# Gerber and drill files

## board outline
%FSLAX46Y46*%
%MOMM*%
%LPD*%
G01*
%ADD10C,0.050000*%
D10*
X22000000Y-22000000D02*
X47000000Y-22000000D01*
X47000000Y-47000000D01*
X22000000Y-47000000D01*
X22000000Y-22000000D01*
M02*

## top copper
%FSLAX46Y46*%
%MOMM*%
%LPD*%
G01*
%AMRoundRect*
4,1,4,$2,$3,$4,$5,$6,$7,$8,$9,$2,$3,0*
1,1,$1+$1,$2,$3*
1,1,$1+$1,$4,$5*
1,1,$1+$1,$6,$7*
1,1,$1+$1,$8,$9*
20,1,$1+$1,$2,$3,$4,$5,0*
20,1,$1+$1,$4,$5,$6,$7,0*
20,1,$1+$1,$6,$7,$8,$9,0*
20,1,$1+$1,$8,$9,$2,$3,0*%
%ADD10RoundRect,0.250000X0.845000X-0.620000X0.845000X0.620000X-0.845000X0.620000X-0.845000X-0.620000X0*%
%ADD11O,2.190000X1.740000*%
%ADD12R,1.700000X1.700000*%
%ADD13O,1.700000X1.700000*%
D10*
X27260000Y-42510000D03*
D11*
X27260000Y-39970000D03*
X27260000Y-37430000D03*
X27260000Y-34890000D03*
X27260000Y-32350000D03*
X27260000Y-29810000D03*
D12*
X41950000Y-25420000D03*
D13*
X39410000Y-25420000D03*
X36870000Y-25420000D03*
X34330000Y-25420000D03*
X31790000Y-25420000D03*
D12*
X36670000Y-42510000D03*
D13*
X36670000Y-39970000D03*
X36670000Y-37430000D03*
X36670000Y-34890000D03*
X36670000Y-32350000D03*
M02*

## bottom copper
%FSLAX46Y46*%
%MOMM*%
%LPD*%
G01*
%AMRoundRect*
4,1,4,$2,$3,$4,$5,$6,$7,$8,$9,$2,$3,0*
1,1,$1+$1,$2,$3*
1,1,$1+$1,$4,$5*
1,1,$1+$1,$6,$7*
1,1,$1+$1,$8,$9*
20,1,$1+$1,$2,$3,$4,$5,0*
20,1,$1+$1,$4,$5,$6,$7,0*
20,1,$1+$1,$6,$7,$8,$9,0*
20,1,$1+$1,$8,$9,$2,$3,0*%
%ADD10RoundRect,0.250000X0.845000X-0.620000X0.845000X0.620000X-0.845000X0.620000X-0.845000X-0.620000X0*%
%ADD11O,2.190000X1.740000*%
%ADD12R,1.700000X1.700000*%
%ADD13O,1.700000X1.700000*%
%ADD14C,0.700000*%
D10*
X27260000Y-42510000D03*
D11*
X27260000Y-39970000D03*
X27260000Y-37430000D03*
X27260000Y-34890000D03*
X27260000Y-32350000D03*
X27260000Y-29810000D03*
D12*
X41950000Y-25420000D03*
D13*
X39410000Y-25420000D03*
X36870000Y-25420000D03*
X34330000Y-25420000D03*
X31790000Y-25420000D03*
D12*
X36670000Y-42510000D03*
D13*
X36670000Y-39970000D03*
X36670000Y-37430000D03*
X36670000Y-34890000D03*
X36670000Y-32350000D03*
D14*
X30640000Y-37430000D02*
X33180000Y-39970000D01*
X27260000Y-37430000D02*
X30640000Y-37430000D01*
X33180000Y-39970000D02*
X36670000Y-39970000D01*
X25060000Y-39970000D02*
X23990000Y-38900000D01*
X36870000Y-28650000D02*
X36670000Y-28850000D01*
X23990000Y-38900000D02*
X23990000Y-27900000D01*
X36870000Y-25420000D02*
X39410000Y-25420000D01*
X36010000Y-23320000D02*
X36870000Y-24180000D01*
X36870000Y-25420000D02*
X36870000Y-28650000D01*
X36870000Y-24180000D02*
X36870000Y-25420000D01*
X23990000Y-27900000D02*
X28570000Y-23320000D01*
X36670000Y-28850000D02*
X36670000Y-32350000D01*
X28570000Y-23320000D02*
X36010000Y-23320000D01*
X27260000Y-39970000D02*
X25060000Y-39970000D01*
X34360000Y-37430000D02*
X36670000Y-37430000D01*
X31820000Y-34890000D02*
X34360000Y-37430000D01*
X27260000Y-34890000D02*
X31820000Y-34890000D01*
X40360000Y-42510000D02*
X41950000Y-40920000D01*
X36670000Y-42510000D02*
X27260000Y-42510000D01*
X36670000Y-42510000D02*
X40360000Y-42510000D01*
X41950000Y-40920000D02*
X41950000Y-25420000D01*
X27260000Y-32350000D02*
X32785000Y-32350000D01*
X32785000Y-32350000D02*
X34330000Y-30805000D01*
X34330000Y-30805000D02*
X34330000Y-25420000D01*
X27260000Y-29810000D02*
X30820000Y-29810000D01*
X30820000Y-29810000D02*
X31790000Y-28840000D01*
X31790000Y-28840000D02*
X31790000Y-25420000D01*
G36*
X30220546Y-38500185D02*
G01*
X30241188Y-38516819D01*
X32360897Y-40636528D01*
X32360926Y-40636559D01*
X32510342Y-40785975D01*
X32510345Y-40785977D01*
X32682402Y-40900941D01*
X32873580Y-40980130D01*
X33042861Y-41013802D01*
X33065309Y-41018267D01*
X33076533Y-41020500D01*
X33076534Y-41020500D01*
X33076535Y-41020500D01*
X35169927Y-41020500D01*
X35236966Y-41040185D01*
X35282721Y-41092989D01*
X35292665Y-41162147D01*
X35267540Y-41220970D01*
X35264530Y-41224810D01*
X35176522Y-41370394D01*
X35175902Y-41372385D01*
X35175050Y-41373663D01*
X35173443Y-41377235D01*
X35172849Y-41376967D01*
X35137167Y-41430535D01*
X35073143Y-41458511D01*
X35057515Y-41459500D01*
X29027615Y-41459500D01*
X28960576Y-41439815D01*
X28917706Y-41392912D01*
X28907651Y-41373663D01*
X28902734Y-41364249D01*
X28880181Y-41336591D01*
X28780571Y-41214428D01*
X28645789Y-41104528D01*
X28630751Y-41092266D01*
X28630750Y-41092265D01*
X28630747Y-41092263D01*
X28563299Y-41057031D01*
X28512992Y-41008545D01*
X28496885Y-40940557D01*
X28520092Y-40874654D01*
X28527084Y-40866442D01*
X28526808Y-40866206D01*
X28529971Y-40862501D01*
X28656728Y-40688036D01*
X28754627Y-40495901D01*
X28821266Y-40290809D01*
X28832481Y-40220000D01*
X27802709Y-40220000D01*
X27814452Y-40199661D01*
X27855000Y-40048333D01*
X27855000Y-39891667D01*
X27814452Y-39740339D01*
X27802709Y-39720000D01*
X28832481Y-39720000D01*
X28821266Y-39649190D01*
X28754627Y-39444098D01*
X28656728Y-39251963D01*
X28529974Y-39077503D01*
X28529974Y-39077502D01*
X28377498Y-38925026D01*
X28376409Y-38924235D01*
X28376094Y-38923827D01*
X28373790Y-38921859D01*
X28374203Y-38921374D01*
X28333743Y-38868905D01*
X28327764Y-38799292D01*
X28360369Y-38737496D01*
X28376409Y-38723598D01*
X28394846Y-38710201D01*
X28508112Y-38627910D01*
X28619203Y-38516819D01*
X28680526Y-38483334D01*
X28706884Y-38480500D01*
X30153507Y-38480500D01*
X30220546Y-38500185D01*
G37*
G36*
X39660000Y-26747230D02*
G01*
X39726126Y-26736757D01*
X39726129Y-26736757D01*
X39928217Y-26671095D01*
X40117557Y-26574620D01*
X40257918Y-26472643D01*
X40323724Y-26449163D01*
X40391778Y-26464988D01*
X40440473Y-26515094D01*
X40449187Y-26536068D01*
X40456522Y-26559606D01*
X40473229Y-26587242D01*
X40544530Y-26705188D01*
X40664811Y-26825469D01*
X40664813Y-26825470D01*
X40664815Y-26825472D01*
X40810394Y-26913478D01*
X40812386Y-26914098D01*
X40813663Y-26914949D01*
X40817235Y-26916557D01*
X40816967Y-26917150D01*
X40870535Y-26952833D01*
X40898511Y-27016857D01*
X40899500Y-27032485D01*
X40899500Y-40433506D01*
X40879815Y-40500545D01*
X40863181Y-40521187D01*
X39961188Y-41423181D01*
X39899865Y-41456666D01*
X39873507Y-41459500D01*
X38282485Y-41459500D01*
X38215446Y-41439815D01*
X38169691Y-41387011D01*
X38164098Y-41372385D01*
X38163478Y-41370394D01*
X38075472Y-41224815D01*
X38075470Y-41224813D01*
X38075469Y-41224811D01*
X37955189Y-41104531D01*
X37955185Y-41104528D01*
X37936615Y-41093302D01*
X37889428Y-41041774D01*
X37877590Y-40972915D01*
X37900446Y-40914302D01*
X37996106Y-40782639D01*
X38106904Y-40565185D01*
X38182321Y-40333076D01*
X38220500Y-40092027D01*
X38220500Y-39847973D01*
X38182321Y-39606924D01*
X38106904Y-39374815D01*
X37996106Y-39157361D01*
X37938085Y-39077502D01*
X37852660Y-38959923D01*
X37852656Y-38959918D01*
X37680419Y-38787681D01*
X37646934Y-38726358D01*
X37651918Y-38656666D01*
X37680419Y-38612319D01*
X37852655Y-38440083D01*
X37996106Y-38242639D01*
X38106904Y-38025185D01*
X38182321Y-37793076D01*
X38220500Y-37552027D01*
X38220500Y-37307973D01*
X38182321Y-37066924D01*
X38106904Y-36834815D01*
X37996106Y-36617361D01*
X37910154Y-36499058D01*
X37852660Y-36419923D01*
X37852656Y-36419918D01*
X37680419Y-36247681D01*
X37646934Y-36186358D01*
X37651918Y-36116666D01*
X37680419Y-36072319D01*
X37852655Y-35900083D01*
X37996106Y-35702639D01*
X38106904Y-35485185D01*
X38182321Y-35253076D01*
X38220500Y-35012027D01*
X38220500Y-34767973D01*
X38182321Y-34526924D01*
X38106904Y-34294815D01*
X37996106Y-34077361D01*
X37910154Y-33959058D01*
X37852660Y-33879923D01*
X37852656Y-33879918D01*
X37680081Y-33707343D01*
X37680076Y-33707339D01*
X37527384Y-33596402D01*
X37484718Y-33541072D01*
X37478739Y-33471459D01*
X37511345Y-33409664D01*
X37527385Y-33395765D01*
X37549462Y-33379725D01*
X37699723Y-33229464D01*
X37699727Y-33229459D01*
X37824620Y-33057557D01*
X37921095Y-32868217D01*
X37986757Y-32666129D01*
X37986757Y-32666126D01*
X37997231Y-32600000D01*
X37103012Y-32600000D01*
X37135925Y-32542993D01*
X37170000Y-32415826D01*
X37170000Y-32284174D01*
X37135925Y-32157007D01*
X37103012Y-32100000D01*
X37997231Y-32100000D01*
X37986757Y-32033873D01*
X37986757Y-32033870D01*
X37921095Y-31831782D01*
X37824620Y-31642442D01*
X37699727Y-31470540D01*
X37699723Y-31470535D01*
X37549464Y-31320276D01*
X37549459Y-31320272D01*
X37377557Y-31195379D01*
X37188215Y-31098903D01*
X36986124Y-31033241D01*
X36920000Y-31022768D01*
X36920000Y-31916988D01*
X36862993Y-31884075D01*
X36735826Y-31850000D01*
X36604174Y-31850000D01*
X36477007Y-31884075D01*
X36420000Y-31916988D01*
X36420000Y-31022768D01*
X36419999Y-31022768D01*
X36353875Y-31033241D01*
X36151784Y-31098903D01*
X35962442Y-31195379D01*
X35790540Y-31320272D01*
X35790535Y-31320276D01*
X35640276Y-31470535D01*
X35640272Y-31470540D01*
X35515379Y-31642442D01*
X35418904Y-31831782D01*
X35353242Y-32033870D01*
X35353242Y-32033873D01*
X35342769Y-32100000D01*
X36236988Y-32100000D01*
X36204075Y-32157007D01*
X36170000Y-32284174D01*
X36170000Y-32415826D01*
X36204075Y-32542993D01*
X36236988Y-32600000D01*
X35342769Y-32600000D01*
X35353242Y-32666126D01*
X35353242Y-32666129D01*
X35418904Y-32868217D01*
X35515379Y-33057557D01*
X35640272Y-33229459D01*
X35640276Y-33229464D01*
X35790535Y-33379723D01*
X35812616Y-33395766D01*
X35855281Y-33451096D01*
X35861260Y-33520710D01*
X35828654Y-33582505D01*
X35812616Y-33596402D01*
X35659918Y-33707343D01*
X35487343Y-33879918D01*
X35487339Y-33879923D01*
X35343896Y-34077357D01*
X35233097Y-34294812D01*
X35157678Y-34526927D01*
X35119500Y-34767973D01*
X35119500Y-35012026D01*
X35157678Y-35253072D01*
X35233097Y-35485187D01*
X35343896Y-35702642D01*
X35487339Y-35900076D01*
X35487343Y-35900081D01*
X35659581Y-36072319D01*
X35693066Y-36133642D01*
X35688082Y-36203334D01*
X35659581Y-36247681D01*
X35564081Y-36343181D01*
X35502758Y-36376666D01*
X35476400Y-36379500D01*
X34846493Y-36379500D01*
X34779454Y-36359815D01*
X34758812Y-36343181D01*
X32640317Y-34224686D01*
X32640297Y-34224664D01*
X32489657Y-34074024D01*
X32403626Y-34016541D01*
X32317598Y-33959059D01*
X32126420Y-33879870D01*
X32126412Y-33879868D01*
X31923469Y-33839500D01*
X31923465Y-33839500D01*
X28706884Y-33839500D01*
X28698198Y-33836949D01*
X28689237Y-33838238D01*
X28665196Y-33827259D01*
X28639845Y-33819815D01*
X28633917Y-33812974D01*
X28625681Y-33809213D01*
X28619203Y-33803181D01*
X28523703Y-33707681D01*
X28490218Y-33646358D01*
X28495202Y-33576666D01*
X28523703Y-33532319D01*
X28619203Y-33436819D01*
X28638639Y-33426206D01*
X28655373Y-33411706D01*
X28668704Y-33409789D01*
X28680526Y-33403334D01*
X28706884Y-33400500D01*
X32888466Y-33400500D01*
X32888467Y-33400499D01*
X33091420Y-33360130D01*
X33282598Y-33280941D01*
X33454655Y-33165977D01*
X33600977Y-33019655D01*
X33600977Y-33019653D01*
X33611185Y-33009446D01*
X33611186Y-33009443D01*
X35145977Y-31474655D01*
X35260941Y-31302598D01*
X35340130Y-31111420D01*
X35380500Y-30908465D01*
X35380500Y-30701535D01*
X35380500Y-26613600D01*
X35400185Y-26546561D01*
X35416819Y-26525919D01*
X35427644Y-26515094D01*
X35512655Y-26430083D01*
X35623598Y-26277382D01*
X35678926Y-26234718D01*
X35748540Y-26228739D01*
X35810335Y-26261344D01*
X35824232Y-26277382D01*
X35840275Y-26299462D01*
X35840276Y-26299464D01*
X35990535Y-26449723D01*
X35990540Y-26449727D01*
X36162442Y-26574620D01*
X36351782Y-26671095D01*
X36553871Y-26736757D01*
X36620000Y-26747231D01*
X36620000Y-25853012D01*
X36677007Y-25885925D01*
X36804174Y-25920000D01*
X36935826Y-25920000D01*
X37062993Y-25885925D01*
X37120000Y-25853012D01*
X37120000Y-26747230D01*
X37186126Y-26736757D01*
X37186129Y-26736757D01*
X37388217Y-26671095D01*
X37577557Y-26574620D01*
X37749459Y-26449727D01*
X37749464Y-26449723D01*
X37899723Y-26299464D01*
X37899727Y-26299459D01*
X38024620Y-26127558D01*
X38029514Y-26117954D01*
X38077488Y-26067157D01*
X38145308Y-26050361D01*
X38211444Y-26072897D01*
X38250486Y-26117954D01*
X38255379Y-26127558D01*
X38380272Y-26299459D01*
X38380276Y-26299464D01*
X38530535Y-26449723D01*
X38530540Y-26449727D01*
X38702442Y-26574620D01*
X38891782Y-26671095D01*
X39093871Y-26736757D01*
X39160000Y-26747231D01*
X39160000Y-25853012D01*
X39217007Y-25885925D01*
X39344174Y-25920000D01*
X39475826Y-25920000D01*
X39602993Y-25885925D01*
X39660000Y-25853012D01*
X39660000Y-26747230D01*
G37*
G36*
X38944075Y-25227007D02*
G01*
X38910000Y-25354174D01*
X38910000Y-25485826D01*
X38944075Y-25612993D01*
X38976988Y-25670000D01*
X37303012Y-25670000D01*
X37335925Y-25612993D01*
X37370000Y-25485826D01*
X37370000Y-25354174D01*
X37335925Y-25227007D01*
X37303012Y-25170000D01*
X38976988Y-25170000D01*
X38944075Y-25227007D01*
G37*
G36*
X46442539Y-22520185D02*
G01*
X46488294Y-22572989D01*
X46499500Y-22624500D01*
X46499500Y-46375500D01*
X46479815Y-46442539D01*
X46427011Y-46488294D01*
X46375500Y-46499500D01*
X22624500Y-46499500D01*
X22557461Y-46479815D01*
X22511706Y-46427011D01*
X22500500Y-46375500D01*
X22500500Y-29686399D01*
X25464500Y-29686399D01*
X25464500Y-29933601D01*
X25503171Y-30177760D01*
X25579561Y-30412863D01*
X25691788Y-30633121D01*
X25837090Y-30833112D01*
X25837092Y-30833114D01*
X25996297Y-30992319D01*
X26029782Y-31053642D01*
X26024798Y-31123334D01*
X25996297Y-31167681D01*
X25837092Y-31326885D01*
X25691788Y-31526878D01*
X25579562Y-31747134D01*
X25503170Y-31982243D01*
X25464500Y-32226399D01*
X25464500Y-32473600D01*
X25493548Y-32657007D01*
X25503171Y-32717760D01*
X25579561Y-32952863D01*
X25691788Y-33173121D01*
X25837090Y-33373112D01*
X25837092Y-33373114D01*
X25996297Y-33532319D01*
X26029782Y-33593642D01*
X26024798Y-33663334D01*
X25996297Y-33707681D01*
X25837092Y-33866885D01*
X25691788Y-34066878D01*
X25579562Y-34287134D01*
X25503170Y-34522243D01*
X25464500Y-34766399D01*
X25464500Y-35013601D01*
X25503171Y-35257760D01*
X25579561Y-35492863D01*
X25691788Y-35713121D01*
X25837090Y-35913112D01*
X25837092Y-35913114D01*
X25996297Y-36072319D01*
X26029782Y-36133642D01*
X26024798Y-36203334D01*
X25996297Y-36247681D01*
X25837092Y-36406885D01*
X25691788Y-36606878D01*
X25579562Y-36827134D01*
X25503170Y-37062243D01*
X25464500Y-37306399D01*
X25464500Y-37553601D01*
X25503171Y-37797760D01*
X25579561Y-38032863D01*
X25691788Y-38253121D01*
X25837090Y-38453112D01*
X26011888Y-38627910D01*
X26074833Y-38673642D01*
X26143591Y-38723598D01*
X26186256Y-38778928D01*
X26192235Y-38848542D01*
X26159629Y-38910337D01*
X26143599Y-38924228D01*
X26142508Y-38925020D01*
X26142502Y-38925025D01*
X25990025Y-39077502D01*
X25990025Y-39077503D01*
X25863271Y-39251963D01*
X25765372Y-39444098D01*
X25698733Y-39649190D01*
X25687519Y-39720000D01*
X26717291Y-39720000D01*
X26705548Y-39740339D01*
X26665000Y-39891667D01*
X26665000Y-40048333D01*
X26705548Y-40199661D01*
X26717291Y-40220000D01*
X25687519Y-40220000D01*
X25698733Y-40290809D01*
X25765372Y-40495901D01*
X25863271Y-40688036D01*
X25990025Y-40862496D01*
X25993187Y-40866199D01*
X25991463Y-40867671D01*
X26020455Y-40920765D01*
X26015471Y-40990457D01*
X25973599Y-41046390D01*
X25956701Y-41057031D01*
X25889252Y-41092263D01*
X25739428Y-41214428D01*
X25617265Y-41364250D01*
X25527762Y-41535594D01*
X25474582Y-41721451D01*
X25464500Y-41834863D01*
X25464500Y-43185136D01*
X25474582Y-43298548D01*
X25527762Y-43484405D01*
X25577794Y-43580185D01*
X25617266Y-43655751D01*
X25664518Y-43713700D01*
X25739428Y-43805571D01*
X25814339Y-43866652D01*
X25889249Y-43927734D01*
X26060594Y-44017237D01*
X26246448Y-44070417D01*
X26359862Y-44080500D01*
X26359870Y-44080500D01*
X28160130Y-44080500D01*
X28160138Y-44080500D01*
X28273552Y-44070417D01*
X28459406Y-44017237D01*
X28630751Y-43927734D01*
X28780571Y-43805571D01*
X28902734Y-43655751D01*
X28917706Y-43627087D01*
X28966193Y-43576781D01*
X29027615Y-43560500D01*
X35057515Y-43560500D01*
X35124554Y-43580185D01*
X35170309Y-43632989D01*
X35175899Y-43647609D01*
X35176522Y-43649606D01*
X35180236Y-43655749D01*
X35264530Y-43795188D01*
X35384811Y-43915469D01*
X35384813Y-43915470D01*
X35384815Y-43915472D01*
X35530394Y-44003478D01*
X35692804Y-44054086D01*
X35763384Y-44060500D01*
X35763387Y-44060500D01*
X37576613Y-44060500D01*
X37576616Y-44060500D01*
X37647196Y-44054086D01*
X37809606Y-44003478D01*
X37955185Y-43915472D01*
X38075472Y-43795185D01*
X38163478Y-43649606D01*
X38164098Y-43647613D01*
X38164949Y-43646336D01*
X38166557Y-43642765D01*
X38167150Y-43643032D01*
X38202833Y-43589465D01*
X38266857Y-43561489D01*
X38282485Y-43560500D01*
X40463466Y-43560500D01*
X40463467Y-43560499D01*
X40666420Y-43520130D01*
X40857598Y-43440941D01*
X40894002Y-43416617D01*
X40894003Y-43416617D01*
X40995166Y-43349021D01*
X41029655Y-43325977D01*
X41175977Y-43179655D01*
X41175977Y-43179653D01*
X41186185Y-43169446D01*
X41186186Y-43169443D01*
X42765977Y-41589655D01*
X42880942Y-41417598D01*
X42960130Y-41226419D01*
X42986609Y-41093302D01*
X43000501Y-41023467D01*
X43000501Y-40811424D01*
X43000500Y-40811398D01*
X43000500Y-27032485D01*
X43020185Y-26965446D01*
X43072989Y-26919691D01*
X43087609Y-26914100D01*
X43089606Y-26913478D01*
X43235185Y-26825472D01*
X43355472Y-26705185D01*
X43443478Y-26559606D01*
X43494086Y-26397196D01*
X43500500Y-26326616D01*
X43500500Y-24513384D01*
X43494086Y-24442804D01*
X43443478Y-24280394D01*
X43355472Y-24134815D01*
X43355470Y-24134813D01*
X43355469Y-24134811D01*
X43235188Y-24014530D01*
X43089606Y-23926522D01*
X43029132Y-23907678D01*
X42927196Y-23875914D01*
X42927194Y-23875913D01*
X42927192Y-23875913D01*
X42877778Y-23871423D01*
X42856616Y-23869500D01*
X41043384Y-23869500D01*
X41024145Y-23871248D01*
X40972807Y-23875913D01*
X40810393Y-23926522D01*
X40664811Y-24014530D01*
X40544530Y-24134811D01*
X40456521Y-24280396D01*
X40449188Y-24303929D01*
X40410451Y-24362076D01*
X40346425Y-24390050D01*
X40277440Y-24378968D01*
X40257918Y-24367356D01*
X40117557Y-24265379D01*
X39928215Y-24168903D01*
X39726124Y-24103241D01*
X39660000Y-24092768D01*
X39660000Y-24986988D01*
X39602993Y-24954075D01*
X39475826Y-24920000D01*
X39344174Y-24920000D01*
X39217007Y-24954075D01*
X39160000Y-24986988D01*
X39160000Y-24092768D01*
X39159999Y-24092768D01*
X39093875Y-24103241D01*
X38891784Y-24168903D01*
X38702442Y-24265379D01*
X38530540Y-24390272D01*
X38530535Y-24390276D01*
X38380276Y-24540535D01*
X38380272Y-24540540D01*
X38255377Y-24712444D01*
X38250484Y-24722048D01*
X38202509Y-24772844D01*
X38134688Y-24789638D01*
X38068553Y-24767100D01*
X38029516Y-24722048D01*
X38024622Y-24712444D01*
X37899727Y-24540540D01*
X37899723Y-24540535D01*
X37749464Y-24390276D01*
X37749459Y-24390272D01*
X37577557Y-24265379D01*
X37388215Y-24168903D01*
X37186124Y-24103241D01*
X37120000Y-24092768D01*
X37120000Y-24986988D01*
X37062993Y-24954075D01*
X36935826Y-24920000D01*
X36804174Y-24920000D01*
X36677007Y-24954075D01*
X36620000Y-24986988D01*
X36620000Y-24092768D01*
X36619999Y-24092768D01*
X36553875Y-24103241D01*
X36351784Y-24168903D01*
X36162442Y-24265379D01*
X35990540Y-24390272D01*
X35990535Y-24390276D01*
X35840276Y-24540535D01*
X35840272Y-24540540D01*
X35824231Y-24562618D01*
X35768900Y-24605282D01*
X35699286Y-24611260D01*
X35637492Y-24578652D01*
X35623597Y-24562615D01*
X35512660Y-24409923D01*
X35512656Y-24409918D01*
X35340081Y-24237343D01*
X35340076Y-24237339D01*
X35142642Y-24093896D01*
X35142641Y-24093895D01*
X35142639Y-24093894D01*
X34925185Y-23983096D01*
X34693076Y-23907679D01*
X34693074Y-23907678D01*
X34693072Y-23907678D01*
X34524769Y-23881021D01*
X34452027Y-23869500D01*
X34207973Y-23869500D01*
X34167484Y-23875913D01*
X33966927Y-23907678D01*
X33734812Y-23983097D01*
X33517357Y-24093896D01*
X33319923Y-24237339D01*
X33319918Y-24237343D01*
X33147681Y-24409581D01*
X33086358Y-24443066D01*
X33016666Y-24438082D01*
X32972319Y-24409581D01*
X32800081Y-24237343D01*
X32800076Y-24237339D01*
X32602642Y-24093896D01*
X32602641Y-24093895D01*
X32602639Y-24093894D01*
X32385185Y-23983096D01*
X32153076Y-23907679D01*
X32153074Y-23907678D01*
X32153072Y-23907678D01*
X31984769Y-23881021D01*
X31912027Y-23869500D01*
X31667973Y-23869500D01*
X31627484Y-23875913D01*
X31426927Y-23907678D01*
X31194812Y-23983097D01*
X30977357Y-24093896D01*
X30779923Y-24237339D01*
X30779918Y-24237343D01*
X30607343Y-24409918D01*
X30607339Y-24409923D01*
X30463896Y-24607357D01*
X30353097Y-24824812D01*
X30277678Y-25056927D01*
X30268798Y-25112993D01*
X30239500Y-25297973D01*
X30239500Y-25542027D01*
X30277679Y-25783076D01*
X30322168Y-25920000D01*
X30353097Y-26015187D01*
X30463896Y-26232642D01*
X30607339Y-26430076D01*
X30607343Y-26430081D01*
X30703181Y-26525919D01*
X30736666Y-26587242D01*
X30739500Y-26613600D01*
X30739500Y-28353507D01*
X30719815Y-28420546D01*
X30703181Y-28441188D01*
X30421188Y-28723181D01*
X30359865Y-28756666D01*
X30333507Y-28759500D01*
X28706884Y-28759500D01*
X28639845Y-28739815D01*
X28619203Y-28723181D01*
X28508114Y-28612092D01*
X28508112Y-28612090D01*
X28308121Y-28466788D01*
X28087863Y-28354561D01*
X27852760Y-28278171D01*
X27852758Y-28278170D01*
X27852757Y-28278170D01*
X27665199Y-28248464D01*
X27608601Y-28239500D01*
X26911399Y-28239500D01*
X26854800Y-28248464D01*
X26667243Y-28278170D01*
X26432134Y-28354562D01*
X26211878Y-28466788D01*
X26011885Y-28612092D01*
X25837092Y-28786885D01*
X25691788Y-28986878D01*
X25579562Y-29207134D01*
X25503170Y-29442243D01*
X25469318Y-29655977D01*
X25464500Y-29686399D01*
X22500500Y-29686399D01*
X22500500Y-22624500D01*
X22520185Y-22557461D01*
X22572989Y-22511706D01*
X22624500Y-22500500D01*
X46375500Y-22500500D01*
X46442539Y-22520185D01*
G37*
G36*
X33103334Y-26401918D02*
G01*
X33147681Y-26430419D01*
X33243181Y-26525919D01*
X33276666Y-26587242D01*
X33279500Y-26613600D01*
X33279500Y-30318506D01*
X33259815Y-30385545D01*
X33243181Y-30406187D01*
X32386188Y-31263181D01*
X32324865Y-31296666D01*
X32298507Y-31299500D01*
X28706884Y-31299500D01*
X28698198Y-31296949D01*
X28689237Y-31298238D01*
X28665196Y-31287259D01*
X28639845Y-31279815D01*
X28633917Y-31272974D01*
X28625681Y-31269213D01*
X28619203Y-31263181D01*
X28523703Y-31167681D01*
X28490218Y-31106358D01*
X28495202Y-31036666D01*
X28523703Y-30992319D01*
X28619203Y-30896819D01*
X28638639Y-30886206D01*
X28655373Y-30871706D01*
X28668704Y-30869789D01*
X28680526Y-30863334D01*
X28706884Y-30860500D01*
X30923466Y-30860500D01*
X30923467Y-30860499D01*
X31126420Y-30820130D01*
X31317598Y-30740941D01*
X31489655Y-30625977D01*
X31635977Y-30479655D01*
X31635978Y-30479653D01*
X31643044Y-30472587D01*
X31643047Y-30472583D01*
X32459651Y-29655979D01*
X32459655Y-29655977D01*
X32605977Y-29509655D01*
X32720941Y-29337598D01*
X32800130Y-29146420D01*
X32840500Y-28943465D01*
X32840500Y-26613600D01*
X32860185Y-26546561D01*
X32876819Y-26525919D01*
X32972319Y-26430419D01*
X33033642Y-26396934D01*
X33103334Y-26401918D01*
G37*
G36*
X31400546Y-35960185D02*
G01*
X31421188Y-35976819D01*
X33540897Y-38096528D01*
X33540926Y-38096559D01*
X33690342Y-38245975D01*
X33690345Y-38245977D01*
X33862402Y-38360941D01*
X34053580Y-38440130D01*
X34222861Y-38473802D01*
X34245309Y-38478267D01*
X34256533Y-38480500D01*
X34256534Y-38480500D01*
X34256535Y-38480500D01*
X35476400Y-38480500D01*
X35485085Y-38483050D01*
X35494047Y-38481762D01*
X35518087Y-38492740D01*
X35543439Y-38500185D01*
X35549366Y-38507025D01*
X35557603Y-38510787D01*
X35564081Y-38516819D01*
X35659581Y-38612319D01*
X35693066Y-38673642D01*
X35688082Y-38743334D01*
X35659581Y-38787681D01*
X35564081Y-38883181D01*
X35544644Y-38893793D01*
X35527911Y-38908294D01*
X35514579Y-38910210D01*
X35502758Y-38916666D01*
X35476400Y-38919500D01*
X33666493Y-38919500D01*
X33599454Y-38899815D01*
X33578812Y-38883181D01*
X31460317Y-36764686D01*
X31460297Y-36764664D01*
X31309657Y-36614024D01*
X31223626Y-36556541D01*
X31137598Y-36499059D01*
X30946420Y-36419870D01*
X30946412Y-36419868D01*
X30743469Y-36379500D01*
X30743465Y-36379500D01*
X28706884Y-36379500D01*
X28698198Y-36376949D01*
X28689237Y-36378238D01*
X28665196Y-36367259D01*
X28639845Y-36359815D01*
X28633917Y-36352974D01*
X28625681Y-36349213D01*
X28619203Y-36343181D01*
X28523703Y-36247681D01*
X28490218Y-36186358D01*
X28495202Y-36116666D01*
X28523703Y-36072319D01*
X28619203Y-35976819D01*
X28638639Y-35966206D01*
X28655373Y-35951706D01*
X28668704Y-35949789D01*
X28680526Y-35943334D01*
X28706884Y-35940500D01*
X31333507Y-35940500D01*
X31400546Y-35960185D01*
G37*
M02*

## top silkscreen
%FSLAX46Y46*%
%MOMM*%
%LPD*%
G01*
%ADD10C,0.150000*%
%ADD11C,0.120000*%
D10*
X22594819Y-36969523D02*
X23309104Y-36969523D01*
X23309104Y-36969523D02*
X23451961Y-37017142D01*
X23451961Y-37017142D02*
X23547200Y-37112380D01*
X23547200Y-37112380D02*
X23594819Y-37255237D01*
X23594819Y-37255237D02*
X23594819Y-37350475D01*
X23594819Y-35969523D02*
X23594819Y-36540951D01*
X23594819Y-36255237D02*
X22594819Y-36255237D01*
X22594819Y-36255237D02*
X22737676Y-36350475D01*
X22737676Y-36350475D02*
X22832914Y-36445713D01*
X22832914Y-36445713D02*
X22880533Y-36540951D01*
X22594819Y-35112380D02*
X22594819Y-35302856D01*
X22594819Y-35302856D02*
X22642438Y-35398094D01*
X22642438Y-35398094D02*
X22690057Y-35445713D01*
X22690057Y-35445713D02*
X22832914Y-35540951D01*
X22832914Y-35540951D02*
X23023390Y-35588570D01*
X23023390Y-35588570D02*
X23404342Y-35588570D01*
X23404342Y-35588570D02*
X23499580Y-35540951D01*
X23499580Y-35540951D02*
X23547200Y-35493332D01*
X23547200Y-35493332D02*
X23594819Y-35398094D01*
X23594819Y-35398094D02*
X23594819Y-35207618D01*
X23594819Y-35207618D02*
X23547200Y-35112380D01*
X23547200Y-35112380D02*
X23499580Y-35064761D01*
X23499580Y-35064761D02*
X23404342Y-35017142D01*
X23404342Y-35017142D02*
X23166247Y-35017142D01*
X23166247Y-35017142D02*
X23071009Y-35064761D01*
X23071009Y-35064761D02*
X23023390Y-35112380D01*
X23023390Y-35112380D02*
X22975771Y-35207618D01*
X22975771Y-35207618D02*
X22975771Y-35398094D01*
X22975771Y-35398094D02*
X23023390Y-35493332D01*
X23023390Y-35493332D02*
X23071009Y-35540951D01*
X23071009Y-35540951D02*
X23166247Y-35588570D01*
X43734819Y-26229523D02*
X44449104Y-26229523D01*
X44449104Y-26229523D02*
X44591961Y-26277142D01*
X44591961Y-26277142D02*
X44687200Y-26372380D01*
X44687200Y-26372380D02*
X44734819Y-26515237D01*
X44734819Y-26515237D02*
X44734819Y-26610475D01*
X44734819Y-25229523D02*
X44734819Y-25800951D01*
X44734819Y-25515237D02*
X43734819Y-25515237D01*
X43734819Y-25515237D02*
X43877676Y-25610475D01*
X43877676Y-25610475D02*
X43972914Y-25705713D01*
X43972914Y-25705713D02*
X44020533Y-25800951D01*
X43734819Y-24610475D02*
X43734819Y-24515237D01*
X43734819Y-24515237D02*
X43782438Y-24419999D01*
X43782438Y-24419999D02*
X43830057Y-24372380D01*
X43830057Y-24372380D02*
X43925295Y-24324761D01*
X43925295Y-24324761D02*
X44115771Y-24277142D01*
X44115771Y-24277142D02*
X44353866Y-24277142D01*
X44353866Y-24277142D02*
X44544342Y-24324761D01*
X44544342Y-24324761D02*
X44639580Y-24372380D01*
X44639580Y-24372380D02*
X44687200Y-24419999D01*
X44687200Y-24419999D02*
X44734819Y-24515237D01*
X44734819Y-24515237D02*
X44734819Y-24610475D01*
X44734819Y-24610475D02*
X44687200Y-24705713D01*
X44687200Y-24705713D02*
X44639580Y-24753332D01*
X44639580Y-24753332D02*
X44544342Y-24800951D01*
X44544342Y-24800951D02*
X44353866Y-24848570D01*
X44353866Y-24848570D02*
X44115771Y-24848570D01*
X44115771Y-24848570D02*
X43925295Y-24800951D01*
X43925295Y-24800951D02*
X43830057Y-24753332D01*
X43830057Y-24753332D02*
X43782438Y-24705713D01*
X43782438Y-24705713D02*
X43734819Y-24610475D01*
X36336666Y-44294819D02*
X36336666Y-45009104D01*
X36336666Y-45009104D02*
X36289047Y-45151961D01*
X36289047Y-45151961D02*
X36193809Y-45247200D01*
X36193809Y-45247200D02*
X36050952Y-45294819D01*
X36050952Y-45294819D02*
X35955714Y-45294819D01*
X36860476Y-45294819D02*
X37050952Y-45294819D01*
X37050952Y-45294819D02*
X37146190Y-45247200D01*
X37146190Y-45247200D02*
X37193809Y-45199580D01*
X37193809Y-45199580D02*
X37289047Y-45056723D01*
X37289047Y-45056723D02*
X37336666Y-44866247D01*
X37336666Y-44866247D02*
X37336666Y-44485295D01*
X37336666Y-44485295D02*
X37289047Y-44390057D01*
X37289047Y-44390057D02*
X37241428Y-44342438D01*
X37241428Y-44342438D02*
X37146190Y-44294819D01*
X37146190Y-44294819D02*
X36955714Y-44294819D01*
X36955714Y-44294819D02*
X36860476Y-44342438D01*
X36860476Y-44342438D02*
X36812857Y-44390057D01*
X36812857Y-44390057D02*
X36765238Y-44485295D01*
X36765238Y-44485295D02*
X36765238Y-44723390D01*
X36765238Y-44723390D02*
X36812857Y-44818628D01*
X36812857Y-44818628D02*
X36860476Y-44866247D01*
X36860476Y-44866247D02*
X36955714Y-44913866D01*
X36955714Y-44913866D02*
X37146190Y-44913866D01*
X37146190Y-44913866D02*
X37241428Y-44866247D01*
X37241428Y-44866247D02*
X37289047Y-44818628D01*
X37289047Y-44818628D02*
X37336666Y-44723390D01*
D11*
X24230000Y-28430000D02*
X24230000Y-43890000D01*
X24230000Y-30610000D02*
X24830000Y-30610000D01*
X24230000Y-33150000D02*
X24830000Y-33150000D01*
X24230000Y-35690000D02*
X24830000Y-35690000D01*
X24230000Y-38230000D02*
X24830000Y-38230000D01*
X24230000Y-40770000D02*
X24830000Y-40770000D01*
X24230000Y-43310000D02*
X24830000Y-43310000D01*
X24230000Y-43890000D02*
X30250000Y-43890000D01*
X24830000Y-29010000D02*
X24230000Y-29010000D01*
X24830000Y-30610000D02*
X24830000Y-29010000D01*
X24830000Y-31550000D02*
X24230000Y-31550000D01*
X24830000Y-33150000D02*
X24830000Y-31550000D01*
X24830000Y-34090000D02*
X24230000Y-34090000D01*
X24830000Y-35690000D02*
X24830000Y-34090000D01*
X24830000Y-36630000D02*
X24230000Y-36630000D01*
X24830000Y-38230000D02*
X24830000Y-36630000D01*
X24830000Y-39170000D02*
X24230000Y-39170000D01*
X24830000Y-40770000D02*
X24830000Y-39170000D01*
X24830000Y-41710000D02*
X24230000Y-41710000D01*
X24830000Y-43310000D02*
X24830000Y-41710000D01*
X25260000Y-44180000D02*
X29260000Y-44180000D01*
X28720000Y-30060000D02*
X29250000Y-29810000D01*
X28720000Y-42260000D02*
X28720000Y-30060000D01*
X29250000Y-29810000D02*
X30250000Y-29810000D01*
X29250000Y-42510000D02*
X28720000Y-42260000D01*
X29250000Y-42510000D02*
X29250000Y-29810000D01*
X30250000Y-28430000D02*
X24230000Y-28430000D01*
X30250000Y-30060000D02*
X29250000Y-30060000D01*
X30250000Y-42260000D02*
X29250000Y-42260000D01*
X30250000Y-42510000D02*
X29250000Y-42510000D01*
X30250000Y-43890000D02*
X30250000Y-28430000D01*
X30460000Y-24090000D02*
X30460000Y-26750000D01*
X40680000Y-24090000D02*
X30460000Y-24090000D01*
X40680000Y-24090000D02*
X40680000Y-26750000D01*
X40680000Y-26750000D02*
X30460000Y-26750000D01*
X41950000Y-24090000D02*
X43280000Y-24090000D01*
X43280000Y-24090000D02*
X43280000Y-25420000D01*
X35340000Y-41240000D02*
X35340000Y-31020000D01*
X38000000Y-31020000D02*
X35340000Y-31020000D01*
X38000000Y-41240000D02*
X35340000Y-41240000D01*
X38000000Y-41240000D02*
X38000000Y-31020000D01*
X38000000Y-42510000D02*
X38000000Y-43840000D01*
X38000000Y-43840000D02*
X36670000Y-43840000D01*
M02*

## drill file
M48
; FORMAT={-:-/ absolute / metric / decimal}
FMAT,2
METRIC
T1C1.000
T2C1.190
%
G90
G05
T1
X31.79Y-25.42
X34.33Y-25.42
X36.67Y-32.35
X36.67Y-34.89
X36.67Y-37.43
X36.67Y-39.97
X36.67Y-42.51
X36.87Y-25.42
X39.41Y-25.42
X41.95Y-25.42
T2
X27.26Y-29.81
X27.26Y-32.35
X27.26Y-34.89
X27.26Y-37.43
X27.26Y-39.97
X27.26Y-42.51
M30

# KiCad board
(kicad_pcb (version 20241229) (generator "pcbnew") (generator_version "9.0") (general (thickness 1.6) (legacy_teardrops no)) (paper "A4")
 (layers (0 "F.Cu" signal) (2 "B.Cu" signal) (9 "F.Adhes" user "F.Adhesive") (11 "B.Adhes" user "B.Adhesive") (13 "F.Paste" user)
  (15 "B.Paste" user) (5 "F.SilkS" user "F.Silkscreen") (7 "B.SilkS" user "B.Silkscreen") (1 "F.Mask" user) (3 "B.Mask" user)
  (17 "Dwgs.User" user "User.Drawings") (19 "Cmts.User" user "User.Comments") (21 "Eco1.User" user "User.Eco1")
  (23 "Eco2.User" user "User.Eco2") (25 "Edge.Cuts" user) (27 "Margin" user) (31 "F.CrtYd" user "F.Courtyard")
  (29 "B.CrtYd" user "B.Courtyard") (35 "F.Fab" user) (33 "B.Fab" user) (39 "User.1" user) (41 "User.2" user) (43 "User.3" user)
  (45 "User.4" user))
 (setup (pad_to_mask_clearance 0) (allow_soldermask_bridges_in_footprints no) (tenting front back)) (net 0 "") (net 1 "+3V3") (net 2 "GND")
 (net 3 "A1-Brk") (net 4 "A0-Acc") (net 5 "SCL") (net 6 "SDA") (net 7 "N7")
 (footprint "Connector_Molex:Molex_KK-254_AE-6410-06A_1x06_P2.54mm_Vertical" (layer "F.Cu") (at 27.26 42.51 90)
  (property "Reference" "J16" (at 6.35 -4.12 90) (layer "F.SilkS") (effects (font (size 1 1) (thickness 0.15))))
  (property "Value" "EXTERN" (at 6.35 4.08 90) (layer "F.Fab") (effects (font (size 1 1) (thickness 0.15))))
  (fp_line (start 14.08 -3.03) (end -1.38 -3.03) (stroke (width 0.12) (type solid)) (layer "F.SilkS"))
  (fp_line (start 11.9 -3.03) (end 11.9 -2.43) (stroke (width 0.12) (type solid)) (layer "F.SilkS"))
  (fp_line (start 9.36 -3.03) (end 9.36 -2.43) (stroke (width 0.12) (type solid)) (layer "F.SilkS"))
  (fp_line (start 6.82 -3.03) (end 6.82 -2.43) (stroke (width 0.12) (type solid)) (layer "F.SilkS"))
  (fp_line (start 4.28 -3.03) (end 4.28 -2.43) (stroke (width 0.12) (type solid)) (layer "F.SilkS"))
  (fp_line (start 1.74 -3.03) (end 1.74 -2.43) (stroke (width 0.12) (type solid)) (layer "F.SilkS"))
  (fp_line (start -0.8 -3.03) (end -0.8 -2.43) (stroke (width 0.12) (type solid)) (layer "F.SilkS"))
  (fp_line (start -1.38 -3.03) (end -1.38 2.99) (stroke (width 0.12) (type solid)) (layer "F.SilkS"))
  (fp_line (start 13.5 -2.43) (end 13.5 -3.03) (stroke (width 0.12) (type solid)) (layer "F.SilkS"))
  (fp_line (start 11.9 -2.43) (end 13.5 -2.43) (stroke (width 0.12) (type solid)) (layer "F.SilkS"))
  (fp_line (start 10.96 -2.43) (end 10.96 -3.03) (stroke (width 0.12) (type solid)) (layer "F.SilkS"))
  (fp_line (start 9.36 -2.43) (end 10.96 -2.43) (stroke (width 0.12) (type solid)) (layer "F.SilkS"))
  (fp_line (start 8.42 -2.43) (end 8.42 -3.03) (stroke (width 0.12) (type solid)) (layer "F.SilkS"))
  (fp_line (start 6.82 -2.43) (end 8.42 -2.43) (stroke (width 0.12) (type solid)) (layer "F.SilkS"))
  (fp_line (start 5.88 -2.43) (end 5.88 -3.03) (stroke (width 0.12) (type solid)) (layer "F.SilkS"))
  (fp_line (start 4.28 -2.43) (end 5.88 -2.43) (stroke (width 0.12) (type solid)) (layer "F.SilkS"))
  (fp_line (start 3.34 -2.43) (end 3.34 -3.03) (stroke (width 0.12) (type solid)) (layer "F.SilkS"))
  (fp_line (start 1.74 -2.43) (end 3.34 -2.43) (stroke (width 0.12) (type solid)) (layer "F.SilkS"))
  (fp_line (start 0.8 -2.43) (end 0.8 -3.03) (stroke (width 0.12) (type solid)) (layer "F.SilkS"))
  (fp_line (start -0.8 -2.43) (end 0.8 -2.43) (stroke (width 0.12) (type solid)) (layer "F.SilkS"))
  (fp_line (start -1.67 -2) (end -1.67 2) (stroke (width 0.12) (type solid)) (layer "F.SilkS"))
  (fp_line (start 12.45 1.46) (end 12.7 1.99) (stroke (width 0.12) (type solid)) (layer "F.SilkS"))
  (fp_line (start 0.25 1.46) (end 12.45 1.46) (stroke (width 0.12) (type solid)) (layer "F.SilkS"))
  (fp_line (start 12.7 1.99) (end 12.7 2.99) (stroke (width 0.12) (type solid)) (layer "F.SilkS"))
  (fp_line (start 0 1.99) (end 0.25 1.46) (stroke (width 0.12) (type solid)) (layer "F.SilkS"))
  (fp_line (start 0 1.99) (end 12.7 1.99) (stroke (width 0.12) (type solid)) (layer "F.SilkS"))
  (fp_line (start 14.08 2.99) (end 14.08 -3.03) (stroke (width 0.12) (type solid)) (layer "F.SilkS"))
  (fp_line (start 12.45 2.99) (end 12.45 1.99) (stroke (width 0.12) (type solid)) (layer "F.SilkS"))
  (fp_line (start 0.25 2.99) (end 0.25 1.99) (stroke (width 0.12) (type solid)) (layer "F.SilkS"))
  (fp_line (start 0 2.99) (end 0 1.99) (stroke (width 0.12) (type solid)) (layer "F.SilkS"))
  (fp_line (start -1.38 2.99) (end 14.08 2.99) (stroke (width 0.12) (type solid)) (layer "F.SilkS"))
  (pad "1" thru_hole roundrect (at 0 0 90) (size 1.74 2.19) (drill 1.19) (layers "*.Cu" "*.Mask") (remove_unused_layers no)
   (roundrect_rratio 0.143678) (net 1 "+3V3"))
  (pad "2" thru_hole oval (at 2.54 0 90) (size 1.74 2.19) (drill 1.19) (layers "*.Cu" "*.Mask") (remove_unused_layers no) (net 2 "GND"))
  (pad "3" thru_hole oval (at 5.08 0 90) (size 1.74 2.19) (drill 1.19) (layers "*.Cu" "*.Mask") (remove_unused_layers no) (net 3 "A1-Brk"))
  (pad "4" thru_hole oval (at 7.62 0 90) (size 1.74 2.19) (drill 1.19) (layers "*.Cu" "*.Mask") (remove_unused_layers no) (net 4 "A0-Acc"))
  (pad "5" thru_hole oval (at 10.16 0 90) (size 1.74 2.19) (drill 1.19) (layers "*.Cu" "*.Mask") (remove_unused_layers no) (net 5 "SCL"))
  (pad "6" thru_hole oval (at 12.7 0 90) (size 1.74 2.19) (drill 1.19) (layers "*.Cu" "*.Mask") (remove_unused_layers no) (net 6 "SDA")))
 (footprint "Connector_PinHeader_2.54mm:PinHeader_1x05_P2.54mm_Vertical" (layer "F.Cu") (at 41.95 25.42 -90)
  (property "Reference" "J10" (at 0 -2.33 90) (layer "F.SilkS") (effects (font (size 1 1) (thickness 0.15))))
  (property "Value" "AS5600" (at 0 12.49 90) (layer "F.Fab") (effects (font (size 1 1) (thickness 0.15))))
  (fp_line (start -1.33 11.49) (end 1.33 11.49) (stroke (width 0.12) (type solid)) (layer "F.SilkS"))
  (fp_line (start -1.33 1.27) (end -1.33 11.49) (stroke (width 0.12) (type solid)) (layer "F.SilkS"))
  (fp_line (start -1.33 1.27) (end 1.33 1.27) (stroke (width 0.12) (type solid)) (layer "F.SilkS"))
  (fp_line (start 1.33 1.27) (end 1.33 11.49) (stroke (width 0.12) (type solid)) (layer "F.SilkS"))
  (fp_line (start -1.33 0) (end -1.33 -1.33) (stroke (width 0.12) (type solid)) (layer "F.SilkS"))
  (fp_line (start -1.33 -1.33) (end 0 -1.33) (stroke (width 0.12) (type solid)) (layer "F.SilkS"))
  (pad "1" thru_hole rect (at 0 0 270) (size 1.7 1.7) (drill 1) (layers "*.Cu" "*.Mask") (remove_unused_layers no) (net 1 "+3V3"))
  (pad "2" thru_hole oval (at 0 2.54 270) (size 1.7 1.7) (drill 1) (layers "*.Cu" "*.Mask") (remove_unused_layers no) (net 2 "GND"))
  (pad "3" thru_hole oval (at 0 5.08 270) (size 1.7 1.7) (drill 1) (layers "*.Cu" "*.Mask") (remove_unused_layers no) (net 2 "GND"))
  (pad "4" thru_hole oval (at 0 7.62 270) (size 1.7 1.7) (drill 1) (layers "*.Cu" "*.Mask") (remove_unused_layers no) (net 5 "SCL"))
  (pad "5" thru_hole oval (at 0 10.16 270) (size 1.7 1.7) (drill 1) (layers "*.Cu" "*.Mask") (remove_unused_layers no) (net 6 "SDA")))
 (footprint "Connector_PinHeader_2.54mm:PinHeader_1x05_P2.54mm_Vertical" (layer "F.Cu") (at 36.67 42.51 180)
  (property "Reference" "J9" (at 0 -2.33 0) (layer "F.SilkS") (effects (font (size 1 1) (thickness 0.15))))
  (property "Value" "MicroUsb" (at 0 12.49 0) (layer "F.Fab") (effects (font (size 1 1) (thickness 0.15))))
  (fp_line (start 1.33 1.27) (end 1.33 11.49) (stroke (width 0.12) (type solid)) (layer "F.SilkS"))
  (fp_line (start -1.33 11.49) (end 1.33 11.49) (stroke (width 0.12) (type solid)) (layer "F.SilkS"))
  (fp_line (start -1.33 1.27) (end 1.33 1.27) (stroke (width 0.12) (type solid)) (layer "F.SilkS"))
  (fp_line (start -1.33 1.27) (end -1.33 11.49) (stroke (width 0.12) (type solid)) (layer "F.SilkS"))
  (fp_line (start -1.33 0) (end -1.33 -1.33) (stroke (width 0.12) (type solid)) (layer "F.SilkS"))
  (fp_line (start -1.33 -1.33) (end 0 -1.33) (stroke (width 0.12) (type solid)) (layer "F.SilkS"))
  (pad "1" thru_hole rect (at 0 0 180) (size 1.7 1.7) (drill 1) (layers "*.Cu" "*.Mask") (remove_unused_layers no) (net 1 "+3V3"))
  (pad "2" thru_hole oval (at 0 2.54 180) (size 1.7 1.7) (drill 1) (layers "*.Cu" "*.Mask") (remove_unused_layers no) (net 3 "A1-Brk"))
  (pad "3" thru_hole oval (at 0 5.08 180) (size 1.7 1.7) (drill 1) (layers "*.Cu" "*.Mask") (remove_unused_layers no) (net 4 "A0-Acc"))
  (pad "4" thru_hole oval (at 0 7.62 180) (size 1.7 1.7) (drill 1) (layers "*.Cu" "*.Mask") (remove_unused_layers no) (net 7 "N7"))
  (pad "5" thru_hole oval (at 0 10.16 180) (size 1.7 1.7) (drill 1) (layers "*.Cu" "*.Mask") (remove_unused_layers no) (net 2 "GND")))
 (gr_rect (start 22 22) (end 47 47) (stroke (width 0.05) (type solid)) (fill no) (layer "Edge.Cuts"))
 (segment (start 30.64 37.43) (end 33.18 39.97) (width 0.7) (layer "B.Cu") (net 3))
 (segment (start 27.26 37.43) (end 30.64 37.43) (width 0.7) (layer "B.Cu") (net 3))
 (segment (start 33.18 39.97) (end 36.67 39.97) (width 0.7) (layer "B.Cu") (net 3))
 (segment (start 25.06 39.97) (end 23.99 38.9) (width 0.7) (layer "B.Cu") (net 2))
 (segment (start 36.87 28.65) (end 36.67 28.85) (width 0.7) (layer "B.Cu") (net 2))
 (segment (start 23.99 38.9) (end 23.99 27.9) (width 0.7) (layer "B.Cu") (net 2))
 (segment (start 36.87 25.42) (end 39.41 25.42) (width 0.7) (layer "B.Cu") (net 2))
 (segment (start 36.01 23.32) (end 36.87 24.18) (width 0.7) (layer "B.Cu") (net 2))
 (segment (start 36.87 25.42) (end 36.87 28.65) (width 0.7) (layer "B.Cu") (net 2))
 (segment (start 36.87 24.18) (end 36.87 25.42) (width 0.7) (layer "B.Cu") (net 2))
 (segment (start 23.99 27.9) (end 28.57 23.32) (width 0.7) (layer "B.Cu") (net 2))
 (segment (start 36.67 28.85) (end 36.67 32.35) (width 0.7) (layer "B.Cu") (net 2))
 (segment (start 28.57 23.32) (end 36.01 23.32) (width 0.7) (layer "B.Cu") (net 2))
 (segment (start 27.26 39.97) (end 25.06 39.97) (width 0.7) (layer "B.Cu") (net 2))
 (segment (start 34.36 37.43) (end 36.67 37.43) (width 0.7) (layer "B.Cu") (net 4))
 (segment (start 31.82 34.89) (end 34.36 37.43) (width 0.7) (layer "B.Cu") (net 4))
 (segment (start 27.26 34.89) (end 31.82 34.89) (width 0.7) (layer "B.Cu") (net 4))
 (segment (start 40.36 42.51) (end 41.95 40.92) (width 0.7) (layer "B.Cu") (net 1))
 (segment (start 36.67 42.51) (end 27.26 42.51) (width 0.7) (layer "B.Cu") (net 1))
 (segment (start 36.67 42.51) (end 40.36 42.51) (width 0.7) (layer "B.Cu") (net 1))
 (segment (start 41.95 40.92) (end 41.95 25.42) (width 0.7) (layer "B.Cu") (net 1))
 (segment (start 27.26 32.35) (end 32.785 32.35) (width 0.7) (layer "B.Cu") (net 5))
 (segment (start 32.785 32.35) (end 34.33 30.805) (width 0.7) (layer "B.Cu") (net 5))
 (segment (start 34.33 30.805) (end 34.33 25.42) (width 0.7) (layer "B.Cu") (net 5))
 (segment (start 27.26 29.81) (end 30.82 29.81) (width 0.7) (layer "B.Cu") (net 6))
 (segment (start 30.82 29.81) (end 31.79 28.84) (width 0.7) (layer "B.Cu") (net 6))
 (segment (start 31.79 28.84) (end 31.79 25.42) (width 0.7) (layer "B.Cu") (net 6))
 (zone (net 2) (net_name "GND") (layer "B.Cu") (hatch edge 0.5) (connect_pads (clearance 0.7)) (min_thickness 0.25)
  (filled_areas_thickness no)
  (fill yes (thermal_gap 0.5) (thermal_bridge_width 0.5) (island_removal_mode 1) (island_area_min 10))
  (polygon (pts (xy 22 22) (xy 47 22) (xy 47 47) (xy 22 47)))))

